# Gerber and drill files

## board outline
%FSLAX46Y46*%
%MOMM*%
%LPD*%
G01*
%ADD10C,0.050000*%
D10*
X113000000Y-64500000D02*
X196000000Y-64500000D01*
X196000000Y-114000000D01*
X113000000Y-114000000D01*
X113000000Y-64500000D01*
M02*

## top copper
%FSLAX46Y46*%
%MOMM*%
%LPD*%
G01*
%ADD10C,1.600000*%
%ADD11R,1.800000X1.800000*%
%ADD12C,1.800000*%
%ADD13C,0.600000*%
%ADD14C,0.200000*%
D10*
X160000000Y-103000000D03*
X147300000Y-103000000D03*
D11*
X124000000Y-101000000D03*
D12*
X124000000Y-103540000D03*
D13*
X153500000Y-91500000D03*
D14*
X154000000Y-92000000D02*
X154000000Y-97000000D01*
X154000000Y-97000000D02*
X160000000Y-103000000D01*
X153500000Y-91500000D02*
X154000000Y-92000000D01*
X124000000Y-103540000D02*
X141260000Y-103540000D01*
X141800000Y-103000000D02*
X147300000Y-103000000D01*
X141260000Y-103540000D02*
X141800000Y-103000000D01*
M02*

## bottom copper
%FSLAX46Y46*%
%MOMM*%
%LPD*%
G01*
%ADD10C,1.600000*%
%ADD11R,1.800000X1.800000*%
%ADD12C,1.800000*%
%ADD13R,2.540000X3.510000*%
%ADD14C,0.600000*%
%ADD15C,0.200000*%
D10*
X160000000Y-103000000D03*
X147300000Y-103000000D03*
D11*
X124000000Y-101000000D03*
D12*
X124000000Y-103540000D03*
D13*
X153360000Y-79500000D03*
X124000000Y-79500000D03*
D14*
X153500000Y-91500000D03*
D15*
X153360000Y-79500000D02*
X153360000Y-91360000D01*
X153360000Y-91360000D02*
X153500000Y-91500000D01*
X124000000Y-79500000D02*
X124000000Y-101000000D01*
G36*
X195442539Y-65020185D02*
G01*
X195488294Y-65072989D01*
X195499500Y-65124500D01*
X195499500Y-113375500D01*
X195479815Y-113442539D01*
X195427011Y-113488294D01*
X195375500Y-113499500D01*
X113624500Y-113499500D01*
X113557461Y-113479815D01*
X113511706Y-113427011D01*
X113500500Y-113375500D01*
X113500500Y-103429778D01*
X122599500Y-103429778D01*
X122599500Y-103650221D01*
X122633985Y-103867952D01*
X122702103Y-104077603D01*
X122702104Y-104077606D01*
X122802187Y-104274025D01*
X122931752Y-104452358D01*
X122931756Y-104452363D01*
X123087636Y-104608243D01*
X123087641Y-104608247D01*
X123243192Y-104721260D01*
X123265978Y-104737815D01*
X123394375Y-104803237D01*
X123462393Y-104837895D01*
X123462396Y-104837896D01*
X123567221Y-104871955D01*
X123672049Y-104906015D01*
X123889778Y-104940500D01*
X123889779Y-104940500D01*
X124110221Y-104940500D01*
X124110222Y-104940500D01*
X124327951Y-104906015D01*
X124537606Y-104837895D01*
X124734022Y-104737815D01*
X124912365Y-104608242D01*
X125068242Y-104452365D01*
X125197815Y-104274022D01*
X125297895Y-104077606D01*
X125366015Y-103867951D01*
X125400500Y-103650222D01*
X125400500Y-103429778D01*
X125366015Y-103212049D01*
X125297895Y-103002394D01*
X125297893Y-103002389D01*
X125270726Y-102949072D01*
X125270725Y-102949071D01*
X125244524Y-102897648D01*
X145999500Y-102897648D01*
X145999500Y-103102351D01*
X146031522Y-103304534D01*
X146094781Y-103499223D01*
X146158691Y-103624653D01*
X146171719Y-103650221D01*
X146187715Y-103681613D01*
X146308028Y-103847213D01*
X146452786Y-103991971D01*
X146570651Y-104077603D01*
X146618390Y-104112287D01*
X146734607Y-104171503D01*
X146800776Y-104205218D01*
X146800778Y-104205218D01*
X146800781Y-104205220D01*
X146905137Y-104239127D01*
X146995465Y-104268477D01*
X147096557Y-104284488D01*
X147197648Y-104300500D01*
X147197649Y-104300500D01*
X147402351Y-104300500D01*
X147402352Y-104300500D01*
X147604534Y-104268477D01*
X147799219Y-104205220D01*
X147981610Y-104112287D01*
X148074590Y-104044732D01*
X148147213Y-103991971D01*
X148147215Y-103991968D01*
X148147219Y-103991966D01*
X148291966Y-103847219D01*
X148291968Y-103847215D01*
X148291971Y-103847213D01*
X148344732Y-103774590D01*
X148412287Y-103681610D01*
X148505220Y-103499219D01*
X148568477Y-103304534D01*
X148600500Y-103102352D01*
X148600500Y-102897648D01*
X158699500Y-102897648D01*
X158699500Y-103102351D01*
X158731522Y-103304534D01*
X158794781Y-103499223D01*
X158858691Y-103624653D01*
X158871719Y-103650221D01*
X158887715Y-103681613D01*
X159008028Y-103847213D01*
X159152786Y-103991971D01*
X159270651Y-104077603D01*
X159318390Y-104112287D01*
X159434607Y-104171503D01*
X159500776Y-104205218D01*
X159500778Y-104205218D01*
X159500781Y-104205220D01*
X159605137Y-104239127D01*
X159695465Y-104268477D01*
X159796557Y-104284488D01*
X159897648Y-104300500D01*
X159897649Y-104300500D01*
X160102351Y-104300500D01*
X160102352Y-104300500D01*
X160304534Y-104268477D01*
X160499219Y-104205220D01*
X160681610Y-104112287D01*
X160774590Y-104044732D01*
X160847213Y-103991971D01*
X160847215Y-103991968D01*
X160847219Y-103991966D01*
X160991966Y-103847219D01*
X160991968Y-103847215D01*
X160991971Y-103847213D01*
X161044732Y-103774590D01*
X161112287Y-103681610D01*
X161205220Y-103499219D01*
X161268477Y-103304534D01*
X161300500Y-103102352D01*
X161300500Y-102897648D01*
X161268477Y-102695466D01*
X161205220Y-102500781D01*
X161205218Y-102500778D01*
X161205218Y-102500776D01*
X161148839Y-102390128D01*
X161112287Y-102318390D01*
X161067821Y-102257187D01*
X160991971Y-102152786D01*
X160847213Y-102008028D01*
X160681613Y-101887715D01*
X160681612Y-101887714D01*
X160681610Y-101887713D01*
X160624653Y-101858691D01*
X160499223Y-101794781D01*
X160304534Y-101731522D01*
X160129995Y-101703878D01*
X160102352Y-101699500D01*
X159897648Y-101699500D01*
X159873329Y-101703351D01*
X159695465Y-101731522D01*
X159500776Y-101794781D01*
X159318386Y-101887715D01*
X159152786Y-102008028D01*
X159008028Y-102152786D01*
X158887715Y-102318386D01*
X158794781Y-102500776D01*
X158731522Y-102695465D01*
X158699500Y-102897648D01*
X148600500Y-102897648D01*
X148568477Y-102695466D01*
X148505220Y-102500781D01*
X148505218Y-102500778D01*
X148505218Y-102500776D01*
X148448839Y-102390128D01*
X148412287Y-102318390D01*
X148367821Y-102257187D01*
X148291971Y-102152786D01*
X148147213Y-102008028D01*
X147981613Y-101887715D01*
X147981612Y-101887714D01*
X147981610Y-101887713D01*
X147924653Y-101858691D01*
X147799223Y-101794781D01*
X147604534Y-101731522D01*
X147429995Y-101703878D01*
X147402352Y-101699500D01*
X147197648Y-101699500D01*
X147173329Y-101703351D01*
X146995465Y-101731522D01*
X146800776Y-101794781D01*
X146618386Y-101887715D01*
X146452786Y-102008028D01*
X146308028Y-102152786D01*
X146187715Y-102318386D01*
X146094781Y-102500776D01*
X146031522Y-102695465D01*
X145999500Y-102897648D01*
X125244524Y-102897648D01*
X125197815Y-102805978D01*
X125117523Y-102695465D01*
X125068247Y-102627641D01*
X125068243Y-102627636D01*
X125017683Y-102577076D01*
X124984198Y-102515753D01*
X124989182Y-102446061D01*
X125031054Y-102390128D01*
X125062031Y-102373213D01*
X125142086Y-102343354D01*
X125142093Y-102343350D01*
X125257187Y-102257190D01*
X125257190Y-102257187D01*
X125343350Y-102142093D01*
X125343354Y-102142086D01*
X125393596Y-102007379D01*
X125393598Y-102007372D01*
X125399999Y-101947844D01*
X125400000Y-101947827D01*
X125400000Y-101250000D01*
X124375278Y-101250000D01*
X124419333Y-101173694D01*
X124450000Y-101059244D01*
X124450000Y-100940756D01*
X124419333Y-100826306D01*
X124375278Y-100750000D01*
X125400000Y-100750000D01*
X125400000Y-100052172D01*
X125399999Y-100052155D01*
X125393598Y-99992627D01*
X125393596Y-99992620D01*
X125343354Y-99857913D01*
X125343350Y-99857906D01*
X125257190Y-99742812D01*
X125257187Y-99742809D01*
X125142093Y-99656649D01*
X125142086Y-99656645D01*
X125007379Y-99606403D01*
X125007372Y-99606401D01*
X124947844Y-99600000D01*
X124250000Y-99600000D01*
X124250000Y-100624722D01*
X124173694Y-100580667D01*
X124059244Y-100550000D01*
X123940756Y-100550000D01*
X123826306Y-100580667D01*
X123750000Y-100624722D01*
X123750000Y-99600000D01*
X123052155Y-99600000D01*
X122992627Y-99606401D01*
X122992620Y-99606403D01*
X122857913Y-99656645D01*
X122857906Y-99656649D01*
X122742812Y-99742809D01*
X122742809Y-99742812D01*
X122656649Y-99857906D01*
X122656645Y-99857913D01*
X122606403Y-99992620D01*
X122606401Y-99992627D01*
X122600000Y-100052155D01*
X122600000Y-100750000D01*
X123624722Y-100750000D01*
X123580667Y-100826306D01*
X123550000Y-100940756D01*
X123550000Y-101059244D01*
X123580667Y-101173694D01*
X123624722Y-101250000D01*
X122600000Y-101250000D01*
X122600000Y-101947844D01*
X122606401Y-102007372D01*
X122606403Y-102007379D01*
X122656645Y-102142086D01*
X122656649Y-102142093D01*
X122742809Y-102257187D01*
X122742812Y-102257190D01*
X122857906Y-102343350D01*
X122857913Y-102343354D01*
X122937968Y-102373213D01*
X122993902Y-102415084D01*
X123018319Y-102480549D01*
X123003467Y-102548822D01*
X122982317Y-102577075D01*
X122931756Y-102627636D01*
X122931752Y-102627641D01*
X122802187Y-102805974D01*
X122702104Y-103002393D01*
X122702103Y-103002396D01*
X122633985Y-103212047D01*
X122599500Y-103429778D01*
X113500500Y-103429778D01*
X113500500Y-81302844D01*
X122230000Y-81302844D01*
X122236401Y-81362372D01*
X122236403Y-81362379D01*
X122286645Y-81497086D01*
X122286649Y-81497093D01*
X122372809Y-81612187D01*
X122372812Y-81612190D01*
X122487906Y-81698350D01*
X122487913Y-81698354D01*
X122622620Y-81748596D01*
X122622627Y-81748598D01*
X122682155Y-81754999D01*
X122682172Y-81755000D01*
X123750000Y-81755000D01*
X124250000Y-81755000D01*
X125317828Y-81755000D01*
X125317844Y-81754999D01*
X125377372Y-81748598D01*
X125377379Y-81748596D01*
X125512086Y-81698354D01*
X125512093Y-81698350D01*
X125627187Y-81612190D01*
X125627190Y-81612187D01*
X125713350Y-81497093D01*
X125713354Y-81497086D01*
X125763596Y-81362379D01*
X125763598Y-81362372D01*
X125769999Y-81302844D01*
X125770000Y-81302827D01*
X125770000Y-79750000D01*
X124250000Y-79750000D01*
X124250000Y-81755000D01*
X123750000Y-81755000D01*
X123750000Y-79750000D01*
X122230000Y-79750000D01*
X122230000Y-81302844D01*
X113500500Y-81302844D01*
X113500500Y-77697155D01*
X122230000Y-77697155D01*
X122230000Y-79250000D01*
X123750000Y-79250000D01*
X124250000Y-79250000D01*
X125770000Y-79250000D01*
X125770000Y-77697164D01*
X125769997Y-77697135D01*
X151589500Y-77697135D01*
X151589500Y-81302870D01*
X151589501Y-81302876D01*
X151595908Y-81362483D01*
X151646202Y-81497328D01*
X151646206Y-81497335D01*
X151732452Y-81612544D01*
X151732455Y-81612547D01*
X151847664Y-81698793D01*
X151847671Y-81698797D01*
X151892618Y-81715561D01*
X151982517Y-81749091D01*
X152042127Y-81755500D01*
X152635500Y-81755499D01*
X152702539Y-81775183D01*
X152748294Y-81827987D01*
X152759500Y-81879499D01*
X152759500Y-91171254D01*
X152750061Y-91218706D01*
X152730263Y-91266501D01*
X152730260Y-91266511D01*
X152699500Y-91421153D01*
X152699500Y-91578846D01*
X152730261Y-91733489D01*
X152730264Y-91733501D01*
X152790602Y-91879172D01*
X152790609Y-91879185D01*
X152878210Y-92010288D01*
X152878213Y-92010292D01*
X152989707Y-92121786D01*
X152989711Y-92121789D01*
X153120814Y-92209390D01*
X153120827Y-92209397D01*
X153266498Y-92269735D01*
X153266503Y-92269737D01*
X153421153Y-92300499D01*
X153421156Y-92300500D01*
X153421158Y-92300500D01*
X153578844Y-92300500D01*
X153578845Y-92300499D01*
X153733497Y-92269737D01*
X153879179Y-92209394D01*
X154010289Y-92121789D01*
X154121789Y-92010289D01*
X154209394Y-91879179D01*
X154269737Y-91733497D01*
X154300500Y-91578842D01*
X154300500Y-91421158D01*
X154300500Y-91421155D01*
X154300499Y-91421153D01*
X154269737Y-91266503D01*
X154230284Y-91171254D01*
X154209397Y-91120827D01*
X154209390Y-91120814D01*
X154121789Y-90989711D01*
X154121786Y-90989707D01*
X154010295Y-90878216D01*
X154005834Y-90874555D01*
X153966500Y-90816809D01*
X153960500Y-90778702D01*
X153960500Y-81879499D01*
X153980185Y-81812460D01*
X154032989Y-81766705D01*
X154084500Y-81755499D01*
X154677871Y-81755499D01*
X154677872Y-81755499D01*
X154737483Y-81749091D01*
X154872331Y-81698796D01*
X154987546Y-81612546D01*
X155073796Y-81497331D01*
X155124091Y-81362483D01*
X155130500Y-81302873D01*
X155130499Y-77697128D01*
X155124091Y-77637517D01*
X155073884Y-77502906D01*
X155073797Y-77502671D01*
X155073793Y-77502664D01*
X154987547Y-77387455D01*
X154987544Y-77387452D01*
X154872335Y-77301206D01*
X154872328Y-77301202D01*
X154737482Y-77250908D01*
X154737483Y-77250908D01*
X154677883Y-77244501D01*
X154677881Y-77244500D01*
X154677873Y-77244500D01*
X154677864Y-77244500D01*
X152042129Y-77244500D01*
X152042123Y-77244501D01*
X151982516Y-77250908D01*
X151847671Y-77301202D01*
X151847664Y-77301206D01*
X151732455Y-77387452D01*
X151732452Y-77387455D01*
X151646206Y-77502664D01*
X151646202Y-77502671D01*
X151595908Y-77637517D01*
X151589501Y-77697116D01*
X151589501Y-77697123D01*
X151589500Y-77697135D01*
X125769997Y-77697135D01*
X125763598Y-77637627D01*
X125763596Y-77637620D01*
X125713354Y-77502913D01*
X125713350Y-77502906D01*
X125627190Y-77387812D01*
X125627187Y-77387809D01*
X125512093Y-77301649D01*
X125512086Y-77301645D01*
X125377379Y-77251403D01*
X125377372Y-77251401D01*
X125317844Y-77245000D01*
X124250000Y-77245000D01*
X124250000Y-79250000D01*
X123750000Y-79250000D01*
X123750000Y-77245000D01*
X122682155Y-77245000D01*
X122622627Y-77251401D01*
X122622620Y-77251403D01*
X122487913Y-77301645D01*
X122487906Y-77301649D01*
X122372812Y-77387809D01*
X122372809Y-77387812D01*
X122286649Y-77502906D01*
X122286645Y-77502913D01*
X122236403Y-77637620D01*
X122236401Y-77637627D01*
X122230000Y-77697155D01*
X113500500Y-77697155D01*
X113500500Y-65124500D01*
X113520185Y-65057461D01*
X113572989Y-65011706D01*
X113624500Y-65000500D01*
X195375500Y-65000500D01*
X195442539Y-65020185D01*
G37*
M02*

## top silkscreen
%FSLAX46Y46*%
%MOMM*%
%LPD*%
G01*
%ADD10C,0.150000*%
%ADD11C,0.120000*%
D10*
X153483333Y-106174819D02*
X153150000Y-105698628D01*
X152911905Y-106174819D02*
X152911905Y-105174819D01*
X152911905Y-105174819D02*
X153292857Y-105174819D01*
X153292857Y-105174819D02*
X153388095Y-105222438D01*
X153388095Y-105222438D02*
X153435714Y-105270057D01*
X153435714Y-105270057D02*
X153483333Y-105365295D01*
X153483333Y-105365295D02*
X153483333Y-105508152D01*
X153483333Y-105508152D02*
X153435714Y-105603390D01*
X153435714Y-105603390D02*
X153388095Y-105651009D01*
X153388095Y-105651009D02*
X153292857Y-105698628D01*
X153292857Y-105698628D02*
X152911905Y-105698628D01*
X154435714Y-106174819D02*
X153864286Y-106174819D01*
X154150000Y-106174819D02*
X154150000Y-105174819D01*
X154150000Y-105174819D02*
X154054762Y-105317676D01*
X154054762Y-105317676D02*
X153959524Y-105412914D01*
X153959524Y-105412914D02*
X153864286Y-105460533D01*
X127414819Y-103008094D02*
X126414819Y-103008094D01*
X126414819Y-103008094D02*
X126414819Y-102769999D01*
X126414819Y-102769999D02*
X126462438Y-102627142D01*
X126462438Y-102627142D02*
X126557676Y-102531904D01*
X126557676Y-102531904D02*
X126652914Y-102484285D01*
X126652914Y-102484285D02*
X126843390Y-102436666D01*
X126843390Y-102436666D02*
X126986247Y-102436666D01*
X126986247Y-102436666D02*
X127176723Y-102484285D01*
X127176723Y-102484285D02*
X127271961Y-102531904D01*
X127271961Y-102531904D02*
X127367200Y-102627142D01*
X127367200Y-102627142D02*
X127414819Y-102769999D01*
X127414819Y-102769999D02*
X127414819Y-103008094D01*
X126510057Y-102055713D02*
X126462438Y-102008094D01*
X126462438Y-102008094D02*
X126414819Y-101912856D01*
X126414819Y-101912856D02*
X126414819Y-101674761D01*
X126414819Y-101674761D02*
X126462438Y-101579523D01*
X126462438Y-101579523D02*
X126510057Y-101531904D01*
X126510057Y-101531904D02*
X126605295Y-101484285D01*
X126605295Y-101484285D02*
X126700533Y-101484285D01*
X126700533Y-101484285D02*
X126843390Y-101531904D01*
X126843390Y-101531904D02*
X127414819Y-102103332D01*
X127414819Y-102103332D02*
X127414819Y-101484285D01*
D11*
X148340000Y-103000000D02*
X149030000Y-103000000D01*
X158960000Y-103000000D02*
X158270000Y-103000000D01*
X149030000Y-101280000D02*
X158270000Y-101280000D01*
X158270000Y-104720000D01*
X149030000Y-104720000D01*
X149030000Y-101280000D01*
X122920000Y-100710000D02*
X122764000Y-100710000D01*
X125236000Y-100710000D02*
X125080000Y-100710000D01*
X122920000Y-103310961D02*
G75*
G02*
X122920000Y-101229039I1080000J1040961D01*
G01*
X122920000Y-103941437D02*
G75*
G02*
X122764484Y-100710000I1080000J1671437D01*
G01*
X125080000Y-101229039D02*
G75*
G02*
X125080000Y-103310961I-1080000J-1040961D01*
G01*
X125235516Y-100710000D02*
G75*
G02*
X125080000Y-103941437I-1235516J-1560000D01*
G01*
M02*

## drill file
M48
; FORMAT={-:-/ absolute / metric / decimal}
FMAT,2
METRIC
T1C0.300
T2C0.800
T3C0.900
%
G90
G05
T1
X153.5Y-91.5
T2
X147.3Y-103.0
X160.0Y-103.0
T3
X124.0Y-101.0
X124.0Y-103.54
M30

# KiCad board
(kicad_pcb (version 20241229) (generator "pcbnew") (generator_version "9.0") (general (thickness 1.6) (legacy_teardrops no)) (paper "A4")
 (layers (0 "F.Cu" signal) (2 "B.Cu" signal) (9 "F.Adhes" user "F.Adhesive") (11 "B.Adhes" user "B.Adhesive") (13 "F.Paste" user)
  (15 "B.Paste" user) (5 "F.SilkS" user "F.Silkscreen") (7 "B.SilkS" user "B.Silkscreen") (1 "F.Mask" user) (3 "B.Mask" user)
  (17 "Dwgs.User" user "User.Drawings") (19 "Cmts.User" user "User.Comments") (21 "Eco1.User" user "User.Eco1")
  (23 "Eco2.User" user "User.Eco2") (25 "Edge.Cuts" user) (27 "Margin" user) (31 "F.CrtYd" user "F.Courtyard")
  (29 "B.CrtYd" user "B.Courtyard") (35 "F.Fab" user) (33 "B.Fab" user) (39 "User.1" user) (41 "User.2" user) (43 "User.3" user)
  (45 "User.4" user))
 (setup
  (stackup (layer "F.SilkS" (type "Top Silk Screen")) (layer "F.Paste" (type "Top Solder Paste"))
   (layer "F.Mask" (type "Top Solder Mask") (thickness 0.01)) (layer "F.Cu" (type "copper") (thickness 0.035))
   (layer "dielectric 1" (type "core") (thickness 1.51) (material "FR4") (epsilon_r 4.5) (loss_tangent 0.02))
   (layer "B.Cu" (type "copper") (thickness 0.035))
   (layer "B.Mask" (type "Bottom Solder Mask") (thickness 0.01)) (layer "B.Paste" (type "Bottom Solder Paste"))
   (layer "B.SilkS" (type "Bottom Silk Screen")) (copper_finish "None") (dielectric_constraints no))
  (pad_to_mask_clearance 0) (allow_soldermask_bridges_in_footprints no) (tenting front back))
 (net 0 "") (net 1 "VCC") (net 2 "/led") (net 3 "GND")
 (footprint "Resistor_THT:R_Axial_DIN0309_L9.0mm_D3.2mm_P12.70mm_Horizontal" (layer "F.Cu") (at 160 103 180)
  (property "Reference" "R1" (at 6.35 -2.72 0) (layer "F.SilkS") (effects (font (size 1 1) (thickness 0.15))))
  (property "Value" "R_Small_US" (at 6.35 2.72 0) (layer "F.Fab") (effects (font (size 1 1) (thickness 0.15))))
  (fp_line (start 11.66 0) (end 10.97 0) (stroke (width 0.12) (type solid)) (layer "F.SilkS"))
  (fp_line (start 1.04 0) (end 1.73 0) (stroke (width 0.12) (type solid)) (layer "F.SilkS"))
  (fp_rect (start 1.73 -1.72) (end 10.97 1.72) (stroke (width 0.12) (type solid)) (fill no) (layer "F.SilkS"))
  (pad "1" thru_hole circle (at 0 0 180) (size 1.6 1.6) (drill 0.8) (layers "*.Cu" "*.Mask") (remove_unused_layers no) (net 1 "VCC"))
  (pad "2" thru_hole circle (at 12.7 0 180) (size 1.6 1.6) (drill 0.8) (layers "*.Cu" "*.Mask") (remove_unused_layers no) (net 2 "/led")))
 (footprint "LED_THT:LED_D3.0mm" (layer "F.Cu") (at 124 101 -90)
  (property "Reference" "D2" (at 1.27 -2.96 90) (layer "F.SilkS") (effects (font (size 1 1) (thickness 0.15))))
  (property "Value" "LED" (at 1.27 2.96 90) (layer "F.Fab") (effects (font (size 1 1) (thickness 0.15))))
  (fp_line (start -0.29 1.08) (end -0.29 1.236) (stroke (width 0.12) (type solid)) (layer "F.SilkS"))
  (fp_line (start -0.29 -1.236) (end -0.29 -1.08) (stroke (width 0.12) (type solid)) (layer "F.SilkS"))
  (fp_arc (start 2.310961 1.08) (mid 1.27 1.5) (end 0.229039 1.08) (stroke (width 0.12) (type solid)) (layer "F.SilkS"))
  (fp_arc (start 2.941437 1.08) (mid 1.36566 1.987699) (end -0.29 1.235516) (stroke (width 0.12) (type solid)) (layer "F.SilkS"))
  (fp_arc (start 0.229039 -1.08) (mid 1.27 -1.5) (end 2.310961 -1.08) (stroke (width 0.12) (type solid)) (layer "F.SilkS"))
  (fp_arc (start -0.29 -1.235516) (mid 1.36566 -1.987699) (end 2.941437 -1.08) (stroke (width 0.12) (type solid)) (layer "F.SilkS"))
  (pad "1" thru_hole rect (at 0 0 270) (size 1.8 1.8) (drill 0.9) (layers "*.Cu" "*.Mask") (remove_unused_layers no) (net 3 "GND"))
  (pad "2" thru_hole circle (at 2.54 0 270) (size 1.8 1.8) (drill 0.9) (layers "*.Cu" "*.Mask") (remove_unused_layers no) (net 2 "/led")))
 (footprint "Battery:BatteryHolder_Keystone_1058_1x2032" (layer "B.Cu") (at 138.68 79.5 180)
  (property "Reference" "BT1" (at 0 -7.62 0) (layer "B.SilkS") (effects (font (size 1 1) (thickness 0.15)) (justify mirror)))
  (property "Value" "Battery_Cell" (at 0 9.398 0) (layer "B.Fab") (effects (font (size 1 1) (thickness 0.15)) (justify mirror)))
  (pad "1" smd rect (at -14.68 0 180) (size 2.54 3.51) (layers "B.Cu" "B.Mask" "B.Paste") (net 1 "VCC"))
  (pad "2" smd rect (at 14.68 0 180) (size 2.54 3.51) (layers "B.Cu" "B.Mask" "B.Paste") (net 3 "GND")))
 (gr_rect (start 113 64.5) (end 196 114) (stroke (width 0.05) (type default)) (fill no) (layer "Edge.Cuts"))
 (segment (start 154 92) (end 154 97) (width 0.2) (layer "F.Cu") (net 1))
 (segment (start 154 97) (end 160 103) (width 0.2) (layer "F.Cu") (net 1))
 (segment (start 153.5 91.5) (end 154 92) (width 0.2) (layer "F.Cu") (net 1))
 (via (at 153.5 91.5) (size 0.6) (drill 0.3) (layers "F.Cu" "B.Cu") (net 1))
 (segment (start 153.36 79.5) (end 153.36 91.36) (width 0.2) (layer "B.Cu") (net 1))
 (segment (start 153.36 91.36) (end 153.5 91.5) (width 0.2) (layer "B.Cu") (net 1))
 (segment (start 124 79.5) (end 124 101) (width 0.2) (layer "B.Cu") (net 3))
 (segment (start 124 103.54) (end 141.26 103.54) (width 0.2) (layer "F.Cu") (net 2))
 (segment (start 141.8 103) (end 147.3 103) (width 0.2) (layer "F.Cu") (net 2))
 (segment (start 141.26 103.54) (end 141.8 103) (width 0.2) (layer "F.Cu") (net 2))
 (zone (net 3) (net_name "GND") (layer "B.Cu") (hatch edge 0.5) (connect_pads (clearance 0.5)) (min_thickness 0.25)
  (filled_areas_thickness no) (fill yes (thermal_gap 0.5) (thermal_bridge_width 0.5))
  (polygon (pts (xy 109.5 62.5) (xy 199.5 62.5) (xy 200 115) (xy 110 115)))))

